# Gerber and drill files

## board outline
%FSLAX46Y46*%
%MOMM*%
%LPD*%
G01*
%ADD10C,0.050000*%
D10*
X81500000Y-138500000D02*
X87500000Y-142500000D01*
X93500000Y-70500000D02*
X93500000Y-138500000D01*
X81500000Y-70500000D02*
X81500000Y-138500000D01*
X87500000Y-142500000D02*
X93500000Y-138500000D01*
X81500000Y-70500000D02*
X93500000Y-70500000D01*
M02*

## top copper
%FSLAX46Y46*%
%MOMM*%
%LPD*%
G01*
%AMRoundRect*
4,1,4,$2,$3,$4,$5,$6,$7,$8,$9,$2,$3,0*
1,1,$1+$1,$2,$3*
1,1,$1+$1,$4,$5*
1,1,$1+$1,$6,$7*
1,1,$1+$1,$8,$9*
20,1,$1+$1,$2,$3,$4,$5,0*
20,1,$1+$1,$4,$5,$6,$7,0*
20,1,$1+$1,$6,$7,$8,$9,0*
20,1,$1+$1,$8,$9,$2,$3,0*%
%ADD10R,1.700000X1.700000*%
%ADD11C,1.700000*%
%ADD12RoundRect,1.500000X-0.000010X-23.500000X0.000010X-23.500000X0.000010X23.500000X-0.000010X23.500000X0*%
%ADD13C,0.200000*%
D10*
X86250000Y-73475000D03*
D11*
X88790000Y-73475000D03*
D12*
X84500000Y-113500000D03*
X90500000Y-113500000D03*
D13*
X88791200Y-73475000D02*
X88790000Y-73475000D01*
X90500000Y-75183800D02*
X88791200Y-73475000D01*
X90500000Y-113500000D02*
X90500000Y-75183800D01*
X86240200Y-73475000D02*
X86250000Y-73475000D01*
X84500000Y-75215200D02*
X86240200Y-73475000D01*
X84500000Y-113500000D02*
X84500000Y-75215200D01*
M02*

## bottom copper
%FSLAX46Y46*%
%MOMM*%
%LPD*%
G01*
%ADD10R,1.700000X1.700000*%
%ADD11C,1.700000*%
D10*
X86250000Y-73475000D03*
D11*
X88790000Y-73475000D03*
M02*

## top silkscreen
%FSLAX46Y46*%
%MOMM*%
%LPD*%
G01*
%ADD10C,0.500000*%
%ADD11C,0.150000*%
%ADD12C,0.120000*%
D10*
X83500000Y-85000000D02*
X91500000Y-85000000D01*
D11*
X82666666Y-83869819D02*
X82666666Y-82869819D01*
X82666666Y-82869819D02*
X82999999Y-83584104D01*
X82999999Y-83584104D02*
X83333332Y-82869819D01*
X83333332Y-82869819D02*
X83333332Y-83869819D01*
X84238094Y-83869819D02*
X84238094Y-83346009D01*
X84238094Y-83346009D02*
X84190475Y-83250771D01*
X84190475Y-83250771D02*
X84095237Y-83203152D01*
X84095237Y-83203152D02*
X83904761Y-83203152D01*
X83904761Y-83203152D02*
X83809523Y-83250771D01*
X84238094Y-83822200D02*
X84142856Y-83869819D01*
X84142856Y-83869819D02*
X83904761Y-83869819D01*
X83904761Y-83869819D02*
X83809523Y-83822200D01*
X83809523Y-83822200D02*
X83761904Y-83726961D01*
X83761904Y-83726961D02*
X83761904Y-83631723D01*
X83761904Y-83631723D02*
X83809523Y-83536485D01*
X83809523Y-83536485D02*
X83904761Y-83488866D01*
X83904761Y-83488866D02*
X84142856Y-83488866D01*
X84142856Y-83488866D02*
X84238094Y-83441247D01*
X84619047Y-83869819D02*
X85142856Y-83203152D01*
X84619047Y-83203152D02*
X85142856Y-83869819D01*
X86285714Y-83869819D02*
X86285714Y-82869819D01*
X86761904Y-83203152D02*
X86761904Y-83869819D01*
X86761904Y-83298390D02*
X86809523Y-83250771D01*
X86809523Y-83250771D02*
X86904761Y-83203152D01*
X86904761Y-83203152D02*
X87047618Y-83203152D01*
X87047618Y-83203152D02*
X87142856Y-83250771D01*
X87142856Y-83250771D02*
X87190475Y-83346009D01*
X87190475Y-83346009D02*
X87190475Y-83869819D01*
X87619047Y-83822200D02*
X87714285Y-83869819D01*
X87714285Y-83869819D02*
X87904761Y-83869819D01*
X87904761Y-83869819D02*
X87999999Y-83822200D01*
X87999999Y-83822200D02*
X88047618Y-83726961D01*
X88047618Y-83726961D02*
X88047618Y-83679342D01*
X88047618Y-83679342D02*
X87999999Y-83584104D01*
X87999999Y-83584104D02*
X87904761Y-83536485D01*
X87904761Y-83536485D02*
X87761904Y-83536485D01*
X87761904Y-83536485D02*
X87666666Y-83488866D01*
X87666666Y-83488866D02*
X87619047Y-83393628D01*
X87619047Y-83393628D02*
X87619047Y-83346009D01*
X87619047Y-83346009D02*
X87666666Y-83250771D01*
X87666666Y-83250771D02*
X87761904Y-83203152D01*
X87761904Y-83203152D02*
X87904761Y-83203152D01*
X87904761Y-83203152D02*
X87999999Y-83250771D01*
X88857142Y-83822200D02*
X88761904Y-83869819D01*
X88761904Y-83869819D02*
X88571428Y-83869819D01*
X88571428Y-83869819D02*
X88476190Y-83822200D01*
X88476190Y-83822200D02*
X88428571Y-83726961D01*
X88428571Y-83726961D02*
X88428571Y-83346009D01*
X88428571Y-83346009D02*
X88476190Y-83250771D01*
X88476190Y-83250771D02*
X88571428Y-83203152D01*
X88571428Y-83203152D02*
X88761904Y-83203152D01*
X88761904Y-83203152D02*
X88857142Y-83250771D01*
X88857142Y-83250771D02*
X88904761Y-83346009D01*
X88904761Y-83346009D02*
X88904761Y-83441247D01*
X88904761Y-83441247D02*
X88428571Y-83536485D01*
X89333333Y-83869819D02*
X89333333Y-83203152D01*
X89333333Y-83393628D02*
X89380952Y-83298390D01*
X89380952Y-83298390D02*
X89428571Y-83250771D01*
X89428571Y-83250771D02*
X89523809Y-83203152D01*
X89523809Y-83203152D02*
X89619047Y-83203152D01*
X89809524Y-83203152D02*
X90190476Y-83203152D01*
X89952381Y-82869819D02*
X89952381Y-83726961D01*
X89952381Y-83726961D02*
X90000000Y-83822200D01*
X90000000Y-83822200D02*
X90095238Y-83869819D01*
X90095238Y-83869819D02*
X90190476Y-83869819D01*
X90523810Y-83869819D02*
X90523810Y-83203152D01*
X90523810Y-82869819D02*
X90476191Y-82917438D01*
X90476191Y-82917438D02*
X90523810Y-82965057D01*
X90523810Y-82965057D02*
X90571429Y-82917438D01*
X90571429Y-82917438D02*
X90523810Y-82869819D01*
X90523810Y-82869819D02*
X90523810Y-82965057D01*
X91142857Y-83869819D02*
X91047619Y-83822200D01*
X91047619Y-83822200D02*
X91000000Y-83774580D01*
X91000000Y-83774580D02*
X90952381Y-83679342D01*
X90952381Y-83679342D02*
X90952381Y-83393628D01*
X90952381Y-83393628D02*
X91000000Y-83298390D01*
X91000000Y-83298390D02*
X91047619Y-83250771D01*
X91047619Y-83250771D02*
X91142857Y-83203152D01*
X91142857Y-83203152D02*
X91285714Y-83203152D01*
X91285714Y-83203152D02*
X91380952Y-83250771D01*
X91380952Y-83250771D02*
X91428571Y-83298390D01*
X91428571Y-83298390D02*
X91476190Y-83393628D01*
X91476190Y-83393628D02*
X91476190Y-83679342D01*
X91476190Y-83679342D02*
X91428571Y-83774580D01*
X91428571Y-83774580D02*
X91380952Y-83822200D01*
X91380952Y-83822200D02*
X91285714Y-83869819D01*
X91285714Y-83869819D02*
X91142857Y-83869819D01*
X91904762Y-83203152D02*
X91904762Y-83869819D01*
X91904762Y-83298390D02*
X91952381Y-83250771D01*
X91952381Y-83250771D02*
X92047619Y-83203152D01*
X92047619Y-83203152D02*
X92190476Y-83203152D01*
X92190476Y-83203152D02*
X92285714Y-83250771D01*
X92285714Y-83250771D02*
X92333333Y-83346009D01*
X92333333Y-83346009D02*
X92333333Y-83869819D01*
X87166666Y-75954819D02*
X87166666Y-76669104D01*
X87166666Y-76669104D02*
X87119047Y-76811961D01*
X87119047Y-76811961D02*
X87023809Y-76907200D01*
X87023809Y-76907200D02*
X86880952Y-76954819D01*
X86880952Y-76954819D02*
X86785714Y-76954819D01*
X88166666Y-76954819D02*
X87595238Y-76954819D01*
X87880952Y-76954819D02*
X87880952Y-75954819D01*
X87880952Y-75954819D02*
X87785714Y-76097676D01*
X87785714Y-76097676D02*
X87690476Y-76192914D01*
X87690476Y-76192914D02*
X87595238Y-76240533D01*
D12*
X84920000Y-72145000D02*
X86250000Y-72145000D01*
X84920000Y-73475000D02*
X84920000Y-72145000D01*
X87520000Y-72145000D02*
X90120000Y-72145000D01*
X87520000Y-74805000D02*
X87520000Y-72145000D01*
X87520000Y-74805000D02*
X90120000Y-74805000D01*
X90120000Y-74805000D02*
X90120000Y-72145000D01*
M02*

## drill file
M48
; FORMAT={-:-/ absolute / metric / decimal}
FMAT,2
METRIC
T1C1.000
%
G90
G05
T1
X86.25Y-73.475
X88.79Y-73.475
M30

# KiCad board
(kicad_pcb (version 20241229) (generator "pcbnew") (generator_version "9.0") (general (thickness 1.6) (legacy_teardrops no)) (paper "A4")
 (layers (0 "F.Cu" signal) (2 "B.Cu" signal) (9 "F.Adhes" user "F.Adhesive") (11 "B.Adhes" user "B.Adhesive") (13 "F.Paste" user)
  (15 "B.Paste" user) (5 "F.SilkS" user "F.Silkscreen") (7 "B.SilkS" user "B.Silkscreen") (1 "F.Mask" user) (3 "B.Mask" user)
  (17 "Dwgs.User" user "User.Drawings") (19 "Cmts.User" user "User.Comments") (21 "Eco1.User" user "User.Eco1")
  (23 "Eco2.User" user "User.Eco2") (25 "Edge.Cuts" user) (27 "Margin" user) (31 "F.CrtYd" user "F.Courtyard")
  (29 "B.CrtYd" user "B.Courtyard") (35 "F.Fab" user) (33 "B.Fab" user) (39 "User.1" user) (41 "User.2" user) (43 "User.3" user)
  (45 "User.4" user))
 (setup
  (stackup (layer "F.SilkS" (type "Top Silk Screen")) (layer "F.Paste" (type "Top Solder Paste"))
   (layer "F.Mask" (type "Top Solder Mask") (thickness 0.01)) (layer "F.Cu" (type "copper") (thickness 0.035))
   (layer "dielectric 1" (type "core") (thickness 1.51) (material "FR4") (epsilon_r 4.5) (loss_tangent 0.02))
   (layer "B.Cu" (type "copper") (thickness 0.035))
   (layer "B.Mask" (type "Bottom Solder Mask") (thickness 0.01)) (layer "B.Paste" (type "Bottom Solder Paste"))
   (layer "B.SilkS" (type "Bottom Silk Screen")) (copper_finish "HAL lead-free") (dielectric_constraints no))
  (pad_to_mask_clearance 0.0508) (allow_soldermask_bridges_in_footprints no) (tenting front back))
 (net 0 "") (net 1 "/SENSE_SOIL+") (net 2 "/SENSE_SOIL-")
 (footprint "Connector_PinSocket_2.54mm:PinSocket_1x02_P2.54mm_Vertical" (layer "F.Cu") (at 86.25 73.475 90)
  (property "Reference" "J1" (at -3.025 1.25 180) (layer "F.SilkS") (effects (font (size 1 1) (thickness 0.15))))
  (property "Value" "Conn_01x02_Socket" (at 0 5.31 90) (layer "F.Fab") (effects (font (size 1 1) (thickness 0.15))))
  (fp_line (start 1.33 -1.33) (end 1.33 0) (stroke (width 0.12) (type solid)) (layer "F.SilkS"))
  (fp_line (start 0 -1.33) (end 1.33 -1.33) (stroke (width 0.12) (type solid)) (layer "F.SilkS"))
  (fp_line (start 1.33 1.27) (end 1.33 3.87) (stroke (width 0.12) (type solid)) (layer "F.SilkS"))
  (fp_line (start -1.33 1.27) (end 1.33 1.27) (stroke (width 0.12) (type solid)) (layer "F.SilkS"))
  (fp_line (start -1.33 1.27) (end -1.33 3.87) (stroke (width 0.12) (type solid)) (layer "F.SilkS"))
  (fp_line (start -1.33 3.87) (end 1.33 3.87) (stroke (width 0.12) (type solid)) (layer "F.SilkS"))
  (pad "1" thru_hole rect (at 0 0 90) (size 1.7 1.7) (drill 1) (layers "*.Cu" "*.Mask") (remove_unused_layers no) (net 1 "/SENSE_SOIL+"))
  (pad "2" thru_hole circle (at 0 2.54 90) (size 1.7 1.7) (drill 1) (layers "*.Cu" "*.Mask") (remove_unused_layers no)
   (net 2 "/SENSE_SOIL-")))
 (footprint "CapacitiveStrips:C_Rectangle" (layer "F.Cu") (at 87.5 88.5)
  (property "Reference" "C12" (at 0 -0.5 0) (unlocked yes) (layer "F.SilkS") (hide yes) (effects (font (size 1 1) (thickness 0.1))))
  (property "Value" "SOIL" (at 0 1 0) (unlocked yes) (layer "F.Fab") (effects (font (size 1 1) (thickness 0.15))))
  (pad "1" smd roundrect (at -3 25) (size 3 50) (layers "F.Cu") (roundrect_rratio 0.5) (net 1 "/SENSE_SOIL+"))
  (pad "2" smd roundrect (at 3 25) (size 3 50) (layers "F.Cu") (roundrect_rratio 0.5) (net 2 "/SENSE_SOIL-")))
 (gr_line (start 83.5 85) (end 91.5 85) (stroke (width 0.5) (type solid)) (layer "F.SilkS"))
 (gr_line (start 81.5 138.5) (end 87.5 142.5) (stroke (width 0.05) (type default)) (layer "Edge.Cuts"))
 (gr_line (start 93.5 70.5) (end 93.5 138.5) (stroke (width 0.05) (type default)) (layer "Edge.Cuts"))
 (gr_line (start 81.5 70.5) (end 81.5 138.5) (stroke (width 0.05) (type default)) (layer "Edge.Cuts"))
 (gr_line (start 87.5 142.5) (end 93.5 138.5) (stroke (width 0.05) (type default)) (layer "Edge.Cuts"))
 (gr_line (start 81.5 70.5) (end 93.5 70.5) (stroke (width 0.05) (type default)) (layer "Edge.Cuts"))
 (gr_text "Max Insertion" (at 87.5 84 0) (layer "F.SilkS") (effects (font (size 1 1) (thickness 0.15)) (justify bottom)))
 (segment (start 88.7912 73.475) (end 88.79 73.475) (width 0.2) (layer "F.Cu") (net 2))
 (segment (start 90.5 75.1838) (end 88.7912 73.475) (width 0.2) (layer "F.Cu") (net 2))
 (segment (start 90.5 113.5) (end 90.5 75.1838) (width 0.2) (layer "F.Cu") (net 2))
 (segment (start 86.2402 73.475) (end 86.25 73.475) (width 0.2) (layer "F.Cu") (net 1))
 (segment (start 84.5 75.2152) (end 86.2402 73.475) (width 0.2) (layer "F.Cu") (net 1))
 (segment (start 84.5 113.5) (end 84.5 75.2152) (width 0.2) (layer "F.Cu") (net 1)))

